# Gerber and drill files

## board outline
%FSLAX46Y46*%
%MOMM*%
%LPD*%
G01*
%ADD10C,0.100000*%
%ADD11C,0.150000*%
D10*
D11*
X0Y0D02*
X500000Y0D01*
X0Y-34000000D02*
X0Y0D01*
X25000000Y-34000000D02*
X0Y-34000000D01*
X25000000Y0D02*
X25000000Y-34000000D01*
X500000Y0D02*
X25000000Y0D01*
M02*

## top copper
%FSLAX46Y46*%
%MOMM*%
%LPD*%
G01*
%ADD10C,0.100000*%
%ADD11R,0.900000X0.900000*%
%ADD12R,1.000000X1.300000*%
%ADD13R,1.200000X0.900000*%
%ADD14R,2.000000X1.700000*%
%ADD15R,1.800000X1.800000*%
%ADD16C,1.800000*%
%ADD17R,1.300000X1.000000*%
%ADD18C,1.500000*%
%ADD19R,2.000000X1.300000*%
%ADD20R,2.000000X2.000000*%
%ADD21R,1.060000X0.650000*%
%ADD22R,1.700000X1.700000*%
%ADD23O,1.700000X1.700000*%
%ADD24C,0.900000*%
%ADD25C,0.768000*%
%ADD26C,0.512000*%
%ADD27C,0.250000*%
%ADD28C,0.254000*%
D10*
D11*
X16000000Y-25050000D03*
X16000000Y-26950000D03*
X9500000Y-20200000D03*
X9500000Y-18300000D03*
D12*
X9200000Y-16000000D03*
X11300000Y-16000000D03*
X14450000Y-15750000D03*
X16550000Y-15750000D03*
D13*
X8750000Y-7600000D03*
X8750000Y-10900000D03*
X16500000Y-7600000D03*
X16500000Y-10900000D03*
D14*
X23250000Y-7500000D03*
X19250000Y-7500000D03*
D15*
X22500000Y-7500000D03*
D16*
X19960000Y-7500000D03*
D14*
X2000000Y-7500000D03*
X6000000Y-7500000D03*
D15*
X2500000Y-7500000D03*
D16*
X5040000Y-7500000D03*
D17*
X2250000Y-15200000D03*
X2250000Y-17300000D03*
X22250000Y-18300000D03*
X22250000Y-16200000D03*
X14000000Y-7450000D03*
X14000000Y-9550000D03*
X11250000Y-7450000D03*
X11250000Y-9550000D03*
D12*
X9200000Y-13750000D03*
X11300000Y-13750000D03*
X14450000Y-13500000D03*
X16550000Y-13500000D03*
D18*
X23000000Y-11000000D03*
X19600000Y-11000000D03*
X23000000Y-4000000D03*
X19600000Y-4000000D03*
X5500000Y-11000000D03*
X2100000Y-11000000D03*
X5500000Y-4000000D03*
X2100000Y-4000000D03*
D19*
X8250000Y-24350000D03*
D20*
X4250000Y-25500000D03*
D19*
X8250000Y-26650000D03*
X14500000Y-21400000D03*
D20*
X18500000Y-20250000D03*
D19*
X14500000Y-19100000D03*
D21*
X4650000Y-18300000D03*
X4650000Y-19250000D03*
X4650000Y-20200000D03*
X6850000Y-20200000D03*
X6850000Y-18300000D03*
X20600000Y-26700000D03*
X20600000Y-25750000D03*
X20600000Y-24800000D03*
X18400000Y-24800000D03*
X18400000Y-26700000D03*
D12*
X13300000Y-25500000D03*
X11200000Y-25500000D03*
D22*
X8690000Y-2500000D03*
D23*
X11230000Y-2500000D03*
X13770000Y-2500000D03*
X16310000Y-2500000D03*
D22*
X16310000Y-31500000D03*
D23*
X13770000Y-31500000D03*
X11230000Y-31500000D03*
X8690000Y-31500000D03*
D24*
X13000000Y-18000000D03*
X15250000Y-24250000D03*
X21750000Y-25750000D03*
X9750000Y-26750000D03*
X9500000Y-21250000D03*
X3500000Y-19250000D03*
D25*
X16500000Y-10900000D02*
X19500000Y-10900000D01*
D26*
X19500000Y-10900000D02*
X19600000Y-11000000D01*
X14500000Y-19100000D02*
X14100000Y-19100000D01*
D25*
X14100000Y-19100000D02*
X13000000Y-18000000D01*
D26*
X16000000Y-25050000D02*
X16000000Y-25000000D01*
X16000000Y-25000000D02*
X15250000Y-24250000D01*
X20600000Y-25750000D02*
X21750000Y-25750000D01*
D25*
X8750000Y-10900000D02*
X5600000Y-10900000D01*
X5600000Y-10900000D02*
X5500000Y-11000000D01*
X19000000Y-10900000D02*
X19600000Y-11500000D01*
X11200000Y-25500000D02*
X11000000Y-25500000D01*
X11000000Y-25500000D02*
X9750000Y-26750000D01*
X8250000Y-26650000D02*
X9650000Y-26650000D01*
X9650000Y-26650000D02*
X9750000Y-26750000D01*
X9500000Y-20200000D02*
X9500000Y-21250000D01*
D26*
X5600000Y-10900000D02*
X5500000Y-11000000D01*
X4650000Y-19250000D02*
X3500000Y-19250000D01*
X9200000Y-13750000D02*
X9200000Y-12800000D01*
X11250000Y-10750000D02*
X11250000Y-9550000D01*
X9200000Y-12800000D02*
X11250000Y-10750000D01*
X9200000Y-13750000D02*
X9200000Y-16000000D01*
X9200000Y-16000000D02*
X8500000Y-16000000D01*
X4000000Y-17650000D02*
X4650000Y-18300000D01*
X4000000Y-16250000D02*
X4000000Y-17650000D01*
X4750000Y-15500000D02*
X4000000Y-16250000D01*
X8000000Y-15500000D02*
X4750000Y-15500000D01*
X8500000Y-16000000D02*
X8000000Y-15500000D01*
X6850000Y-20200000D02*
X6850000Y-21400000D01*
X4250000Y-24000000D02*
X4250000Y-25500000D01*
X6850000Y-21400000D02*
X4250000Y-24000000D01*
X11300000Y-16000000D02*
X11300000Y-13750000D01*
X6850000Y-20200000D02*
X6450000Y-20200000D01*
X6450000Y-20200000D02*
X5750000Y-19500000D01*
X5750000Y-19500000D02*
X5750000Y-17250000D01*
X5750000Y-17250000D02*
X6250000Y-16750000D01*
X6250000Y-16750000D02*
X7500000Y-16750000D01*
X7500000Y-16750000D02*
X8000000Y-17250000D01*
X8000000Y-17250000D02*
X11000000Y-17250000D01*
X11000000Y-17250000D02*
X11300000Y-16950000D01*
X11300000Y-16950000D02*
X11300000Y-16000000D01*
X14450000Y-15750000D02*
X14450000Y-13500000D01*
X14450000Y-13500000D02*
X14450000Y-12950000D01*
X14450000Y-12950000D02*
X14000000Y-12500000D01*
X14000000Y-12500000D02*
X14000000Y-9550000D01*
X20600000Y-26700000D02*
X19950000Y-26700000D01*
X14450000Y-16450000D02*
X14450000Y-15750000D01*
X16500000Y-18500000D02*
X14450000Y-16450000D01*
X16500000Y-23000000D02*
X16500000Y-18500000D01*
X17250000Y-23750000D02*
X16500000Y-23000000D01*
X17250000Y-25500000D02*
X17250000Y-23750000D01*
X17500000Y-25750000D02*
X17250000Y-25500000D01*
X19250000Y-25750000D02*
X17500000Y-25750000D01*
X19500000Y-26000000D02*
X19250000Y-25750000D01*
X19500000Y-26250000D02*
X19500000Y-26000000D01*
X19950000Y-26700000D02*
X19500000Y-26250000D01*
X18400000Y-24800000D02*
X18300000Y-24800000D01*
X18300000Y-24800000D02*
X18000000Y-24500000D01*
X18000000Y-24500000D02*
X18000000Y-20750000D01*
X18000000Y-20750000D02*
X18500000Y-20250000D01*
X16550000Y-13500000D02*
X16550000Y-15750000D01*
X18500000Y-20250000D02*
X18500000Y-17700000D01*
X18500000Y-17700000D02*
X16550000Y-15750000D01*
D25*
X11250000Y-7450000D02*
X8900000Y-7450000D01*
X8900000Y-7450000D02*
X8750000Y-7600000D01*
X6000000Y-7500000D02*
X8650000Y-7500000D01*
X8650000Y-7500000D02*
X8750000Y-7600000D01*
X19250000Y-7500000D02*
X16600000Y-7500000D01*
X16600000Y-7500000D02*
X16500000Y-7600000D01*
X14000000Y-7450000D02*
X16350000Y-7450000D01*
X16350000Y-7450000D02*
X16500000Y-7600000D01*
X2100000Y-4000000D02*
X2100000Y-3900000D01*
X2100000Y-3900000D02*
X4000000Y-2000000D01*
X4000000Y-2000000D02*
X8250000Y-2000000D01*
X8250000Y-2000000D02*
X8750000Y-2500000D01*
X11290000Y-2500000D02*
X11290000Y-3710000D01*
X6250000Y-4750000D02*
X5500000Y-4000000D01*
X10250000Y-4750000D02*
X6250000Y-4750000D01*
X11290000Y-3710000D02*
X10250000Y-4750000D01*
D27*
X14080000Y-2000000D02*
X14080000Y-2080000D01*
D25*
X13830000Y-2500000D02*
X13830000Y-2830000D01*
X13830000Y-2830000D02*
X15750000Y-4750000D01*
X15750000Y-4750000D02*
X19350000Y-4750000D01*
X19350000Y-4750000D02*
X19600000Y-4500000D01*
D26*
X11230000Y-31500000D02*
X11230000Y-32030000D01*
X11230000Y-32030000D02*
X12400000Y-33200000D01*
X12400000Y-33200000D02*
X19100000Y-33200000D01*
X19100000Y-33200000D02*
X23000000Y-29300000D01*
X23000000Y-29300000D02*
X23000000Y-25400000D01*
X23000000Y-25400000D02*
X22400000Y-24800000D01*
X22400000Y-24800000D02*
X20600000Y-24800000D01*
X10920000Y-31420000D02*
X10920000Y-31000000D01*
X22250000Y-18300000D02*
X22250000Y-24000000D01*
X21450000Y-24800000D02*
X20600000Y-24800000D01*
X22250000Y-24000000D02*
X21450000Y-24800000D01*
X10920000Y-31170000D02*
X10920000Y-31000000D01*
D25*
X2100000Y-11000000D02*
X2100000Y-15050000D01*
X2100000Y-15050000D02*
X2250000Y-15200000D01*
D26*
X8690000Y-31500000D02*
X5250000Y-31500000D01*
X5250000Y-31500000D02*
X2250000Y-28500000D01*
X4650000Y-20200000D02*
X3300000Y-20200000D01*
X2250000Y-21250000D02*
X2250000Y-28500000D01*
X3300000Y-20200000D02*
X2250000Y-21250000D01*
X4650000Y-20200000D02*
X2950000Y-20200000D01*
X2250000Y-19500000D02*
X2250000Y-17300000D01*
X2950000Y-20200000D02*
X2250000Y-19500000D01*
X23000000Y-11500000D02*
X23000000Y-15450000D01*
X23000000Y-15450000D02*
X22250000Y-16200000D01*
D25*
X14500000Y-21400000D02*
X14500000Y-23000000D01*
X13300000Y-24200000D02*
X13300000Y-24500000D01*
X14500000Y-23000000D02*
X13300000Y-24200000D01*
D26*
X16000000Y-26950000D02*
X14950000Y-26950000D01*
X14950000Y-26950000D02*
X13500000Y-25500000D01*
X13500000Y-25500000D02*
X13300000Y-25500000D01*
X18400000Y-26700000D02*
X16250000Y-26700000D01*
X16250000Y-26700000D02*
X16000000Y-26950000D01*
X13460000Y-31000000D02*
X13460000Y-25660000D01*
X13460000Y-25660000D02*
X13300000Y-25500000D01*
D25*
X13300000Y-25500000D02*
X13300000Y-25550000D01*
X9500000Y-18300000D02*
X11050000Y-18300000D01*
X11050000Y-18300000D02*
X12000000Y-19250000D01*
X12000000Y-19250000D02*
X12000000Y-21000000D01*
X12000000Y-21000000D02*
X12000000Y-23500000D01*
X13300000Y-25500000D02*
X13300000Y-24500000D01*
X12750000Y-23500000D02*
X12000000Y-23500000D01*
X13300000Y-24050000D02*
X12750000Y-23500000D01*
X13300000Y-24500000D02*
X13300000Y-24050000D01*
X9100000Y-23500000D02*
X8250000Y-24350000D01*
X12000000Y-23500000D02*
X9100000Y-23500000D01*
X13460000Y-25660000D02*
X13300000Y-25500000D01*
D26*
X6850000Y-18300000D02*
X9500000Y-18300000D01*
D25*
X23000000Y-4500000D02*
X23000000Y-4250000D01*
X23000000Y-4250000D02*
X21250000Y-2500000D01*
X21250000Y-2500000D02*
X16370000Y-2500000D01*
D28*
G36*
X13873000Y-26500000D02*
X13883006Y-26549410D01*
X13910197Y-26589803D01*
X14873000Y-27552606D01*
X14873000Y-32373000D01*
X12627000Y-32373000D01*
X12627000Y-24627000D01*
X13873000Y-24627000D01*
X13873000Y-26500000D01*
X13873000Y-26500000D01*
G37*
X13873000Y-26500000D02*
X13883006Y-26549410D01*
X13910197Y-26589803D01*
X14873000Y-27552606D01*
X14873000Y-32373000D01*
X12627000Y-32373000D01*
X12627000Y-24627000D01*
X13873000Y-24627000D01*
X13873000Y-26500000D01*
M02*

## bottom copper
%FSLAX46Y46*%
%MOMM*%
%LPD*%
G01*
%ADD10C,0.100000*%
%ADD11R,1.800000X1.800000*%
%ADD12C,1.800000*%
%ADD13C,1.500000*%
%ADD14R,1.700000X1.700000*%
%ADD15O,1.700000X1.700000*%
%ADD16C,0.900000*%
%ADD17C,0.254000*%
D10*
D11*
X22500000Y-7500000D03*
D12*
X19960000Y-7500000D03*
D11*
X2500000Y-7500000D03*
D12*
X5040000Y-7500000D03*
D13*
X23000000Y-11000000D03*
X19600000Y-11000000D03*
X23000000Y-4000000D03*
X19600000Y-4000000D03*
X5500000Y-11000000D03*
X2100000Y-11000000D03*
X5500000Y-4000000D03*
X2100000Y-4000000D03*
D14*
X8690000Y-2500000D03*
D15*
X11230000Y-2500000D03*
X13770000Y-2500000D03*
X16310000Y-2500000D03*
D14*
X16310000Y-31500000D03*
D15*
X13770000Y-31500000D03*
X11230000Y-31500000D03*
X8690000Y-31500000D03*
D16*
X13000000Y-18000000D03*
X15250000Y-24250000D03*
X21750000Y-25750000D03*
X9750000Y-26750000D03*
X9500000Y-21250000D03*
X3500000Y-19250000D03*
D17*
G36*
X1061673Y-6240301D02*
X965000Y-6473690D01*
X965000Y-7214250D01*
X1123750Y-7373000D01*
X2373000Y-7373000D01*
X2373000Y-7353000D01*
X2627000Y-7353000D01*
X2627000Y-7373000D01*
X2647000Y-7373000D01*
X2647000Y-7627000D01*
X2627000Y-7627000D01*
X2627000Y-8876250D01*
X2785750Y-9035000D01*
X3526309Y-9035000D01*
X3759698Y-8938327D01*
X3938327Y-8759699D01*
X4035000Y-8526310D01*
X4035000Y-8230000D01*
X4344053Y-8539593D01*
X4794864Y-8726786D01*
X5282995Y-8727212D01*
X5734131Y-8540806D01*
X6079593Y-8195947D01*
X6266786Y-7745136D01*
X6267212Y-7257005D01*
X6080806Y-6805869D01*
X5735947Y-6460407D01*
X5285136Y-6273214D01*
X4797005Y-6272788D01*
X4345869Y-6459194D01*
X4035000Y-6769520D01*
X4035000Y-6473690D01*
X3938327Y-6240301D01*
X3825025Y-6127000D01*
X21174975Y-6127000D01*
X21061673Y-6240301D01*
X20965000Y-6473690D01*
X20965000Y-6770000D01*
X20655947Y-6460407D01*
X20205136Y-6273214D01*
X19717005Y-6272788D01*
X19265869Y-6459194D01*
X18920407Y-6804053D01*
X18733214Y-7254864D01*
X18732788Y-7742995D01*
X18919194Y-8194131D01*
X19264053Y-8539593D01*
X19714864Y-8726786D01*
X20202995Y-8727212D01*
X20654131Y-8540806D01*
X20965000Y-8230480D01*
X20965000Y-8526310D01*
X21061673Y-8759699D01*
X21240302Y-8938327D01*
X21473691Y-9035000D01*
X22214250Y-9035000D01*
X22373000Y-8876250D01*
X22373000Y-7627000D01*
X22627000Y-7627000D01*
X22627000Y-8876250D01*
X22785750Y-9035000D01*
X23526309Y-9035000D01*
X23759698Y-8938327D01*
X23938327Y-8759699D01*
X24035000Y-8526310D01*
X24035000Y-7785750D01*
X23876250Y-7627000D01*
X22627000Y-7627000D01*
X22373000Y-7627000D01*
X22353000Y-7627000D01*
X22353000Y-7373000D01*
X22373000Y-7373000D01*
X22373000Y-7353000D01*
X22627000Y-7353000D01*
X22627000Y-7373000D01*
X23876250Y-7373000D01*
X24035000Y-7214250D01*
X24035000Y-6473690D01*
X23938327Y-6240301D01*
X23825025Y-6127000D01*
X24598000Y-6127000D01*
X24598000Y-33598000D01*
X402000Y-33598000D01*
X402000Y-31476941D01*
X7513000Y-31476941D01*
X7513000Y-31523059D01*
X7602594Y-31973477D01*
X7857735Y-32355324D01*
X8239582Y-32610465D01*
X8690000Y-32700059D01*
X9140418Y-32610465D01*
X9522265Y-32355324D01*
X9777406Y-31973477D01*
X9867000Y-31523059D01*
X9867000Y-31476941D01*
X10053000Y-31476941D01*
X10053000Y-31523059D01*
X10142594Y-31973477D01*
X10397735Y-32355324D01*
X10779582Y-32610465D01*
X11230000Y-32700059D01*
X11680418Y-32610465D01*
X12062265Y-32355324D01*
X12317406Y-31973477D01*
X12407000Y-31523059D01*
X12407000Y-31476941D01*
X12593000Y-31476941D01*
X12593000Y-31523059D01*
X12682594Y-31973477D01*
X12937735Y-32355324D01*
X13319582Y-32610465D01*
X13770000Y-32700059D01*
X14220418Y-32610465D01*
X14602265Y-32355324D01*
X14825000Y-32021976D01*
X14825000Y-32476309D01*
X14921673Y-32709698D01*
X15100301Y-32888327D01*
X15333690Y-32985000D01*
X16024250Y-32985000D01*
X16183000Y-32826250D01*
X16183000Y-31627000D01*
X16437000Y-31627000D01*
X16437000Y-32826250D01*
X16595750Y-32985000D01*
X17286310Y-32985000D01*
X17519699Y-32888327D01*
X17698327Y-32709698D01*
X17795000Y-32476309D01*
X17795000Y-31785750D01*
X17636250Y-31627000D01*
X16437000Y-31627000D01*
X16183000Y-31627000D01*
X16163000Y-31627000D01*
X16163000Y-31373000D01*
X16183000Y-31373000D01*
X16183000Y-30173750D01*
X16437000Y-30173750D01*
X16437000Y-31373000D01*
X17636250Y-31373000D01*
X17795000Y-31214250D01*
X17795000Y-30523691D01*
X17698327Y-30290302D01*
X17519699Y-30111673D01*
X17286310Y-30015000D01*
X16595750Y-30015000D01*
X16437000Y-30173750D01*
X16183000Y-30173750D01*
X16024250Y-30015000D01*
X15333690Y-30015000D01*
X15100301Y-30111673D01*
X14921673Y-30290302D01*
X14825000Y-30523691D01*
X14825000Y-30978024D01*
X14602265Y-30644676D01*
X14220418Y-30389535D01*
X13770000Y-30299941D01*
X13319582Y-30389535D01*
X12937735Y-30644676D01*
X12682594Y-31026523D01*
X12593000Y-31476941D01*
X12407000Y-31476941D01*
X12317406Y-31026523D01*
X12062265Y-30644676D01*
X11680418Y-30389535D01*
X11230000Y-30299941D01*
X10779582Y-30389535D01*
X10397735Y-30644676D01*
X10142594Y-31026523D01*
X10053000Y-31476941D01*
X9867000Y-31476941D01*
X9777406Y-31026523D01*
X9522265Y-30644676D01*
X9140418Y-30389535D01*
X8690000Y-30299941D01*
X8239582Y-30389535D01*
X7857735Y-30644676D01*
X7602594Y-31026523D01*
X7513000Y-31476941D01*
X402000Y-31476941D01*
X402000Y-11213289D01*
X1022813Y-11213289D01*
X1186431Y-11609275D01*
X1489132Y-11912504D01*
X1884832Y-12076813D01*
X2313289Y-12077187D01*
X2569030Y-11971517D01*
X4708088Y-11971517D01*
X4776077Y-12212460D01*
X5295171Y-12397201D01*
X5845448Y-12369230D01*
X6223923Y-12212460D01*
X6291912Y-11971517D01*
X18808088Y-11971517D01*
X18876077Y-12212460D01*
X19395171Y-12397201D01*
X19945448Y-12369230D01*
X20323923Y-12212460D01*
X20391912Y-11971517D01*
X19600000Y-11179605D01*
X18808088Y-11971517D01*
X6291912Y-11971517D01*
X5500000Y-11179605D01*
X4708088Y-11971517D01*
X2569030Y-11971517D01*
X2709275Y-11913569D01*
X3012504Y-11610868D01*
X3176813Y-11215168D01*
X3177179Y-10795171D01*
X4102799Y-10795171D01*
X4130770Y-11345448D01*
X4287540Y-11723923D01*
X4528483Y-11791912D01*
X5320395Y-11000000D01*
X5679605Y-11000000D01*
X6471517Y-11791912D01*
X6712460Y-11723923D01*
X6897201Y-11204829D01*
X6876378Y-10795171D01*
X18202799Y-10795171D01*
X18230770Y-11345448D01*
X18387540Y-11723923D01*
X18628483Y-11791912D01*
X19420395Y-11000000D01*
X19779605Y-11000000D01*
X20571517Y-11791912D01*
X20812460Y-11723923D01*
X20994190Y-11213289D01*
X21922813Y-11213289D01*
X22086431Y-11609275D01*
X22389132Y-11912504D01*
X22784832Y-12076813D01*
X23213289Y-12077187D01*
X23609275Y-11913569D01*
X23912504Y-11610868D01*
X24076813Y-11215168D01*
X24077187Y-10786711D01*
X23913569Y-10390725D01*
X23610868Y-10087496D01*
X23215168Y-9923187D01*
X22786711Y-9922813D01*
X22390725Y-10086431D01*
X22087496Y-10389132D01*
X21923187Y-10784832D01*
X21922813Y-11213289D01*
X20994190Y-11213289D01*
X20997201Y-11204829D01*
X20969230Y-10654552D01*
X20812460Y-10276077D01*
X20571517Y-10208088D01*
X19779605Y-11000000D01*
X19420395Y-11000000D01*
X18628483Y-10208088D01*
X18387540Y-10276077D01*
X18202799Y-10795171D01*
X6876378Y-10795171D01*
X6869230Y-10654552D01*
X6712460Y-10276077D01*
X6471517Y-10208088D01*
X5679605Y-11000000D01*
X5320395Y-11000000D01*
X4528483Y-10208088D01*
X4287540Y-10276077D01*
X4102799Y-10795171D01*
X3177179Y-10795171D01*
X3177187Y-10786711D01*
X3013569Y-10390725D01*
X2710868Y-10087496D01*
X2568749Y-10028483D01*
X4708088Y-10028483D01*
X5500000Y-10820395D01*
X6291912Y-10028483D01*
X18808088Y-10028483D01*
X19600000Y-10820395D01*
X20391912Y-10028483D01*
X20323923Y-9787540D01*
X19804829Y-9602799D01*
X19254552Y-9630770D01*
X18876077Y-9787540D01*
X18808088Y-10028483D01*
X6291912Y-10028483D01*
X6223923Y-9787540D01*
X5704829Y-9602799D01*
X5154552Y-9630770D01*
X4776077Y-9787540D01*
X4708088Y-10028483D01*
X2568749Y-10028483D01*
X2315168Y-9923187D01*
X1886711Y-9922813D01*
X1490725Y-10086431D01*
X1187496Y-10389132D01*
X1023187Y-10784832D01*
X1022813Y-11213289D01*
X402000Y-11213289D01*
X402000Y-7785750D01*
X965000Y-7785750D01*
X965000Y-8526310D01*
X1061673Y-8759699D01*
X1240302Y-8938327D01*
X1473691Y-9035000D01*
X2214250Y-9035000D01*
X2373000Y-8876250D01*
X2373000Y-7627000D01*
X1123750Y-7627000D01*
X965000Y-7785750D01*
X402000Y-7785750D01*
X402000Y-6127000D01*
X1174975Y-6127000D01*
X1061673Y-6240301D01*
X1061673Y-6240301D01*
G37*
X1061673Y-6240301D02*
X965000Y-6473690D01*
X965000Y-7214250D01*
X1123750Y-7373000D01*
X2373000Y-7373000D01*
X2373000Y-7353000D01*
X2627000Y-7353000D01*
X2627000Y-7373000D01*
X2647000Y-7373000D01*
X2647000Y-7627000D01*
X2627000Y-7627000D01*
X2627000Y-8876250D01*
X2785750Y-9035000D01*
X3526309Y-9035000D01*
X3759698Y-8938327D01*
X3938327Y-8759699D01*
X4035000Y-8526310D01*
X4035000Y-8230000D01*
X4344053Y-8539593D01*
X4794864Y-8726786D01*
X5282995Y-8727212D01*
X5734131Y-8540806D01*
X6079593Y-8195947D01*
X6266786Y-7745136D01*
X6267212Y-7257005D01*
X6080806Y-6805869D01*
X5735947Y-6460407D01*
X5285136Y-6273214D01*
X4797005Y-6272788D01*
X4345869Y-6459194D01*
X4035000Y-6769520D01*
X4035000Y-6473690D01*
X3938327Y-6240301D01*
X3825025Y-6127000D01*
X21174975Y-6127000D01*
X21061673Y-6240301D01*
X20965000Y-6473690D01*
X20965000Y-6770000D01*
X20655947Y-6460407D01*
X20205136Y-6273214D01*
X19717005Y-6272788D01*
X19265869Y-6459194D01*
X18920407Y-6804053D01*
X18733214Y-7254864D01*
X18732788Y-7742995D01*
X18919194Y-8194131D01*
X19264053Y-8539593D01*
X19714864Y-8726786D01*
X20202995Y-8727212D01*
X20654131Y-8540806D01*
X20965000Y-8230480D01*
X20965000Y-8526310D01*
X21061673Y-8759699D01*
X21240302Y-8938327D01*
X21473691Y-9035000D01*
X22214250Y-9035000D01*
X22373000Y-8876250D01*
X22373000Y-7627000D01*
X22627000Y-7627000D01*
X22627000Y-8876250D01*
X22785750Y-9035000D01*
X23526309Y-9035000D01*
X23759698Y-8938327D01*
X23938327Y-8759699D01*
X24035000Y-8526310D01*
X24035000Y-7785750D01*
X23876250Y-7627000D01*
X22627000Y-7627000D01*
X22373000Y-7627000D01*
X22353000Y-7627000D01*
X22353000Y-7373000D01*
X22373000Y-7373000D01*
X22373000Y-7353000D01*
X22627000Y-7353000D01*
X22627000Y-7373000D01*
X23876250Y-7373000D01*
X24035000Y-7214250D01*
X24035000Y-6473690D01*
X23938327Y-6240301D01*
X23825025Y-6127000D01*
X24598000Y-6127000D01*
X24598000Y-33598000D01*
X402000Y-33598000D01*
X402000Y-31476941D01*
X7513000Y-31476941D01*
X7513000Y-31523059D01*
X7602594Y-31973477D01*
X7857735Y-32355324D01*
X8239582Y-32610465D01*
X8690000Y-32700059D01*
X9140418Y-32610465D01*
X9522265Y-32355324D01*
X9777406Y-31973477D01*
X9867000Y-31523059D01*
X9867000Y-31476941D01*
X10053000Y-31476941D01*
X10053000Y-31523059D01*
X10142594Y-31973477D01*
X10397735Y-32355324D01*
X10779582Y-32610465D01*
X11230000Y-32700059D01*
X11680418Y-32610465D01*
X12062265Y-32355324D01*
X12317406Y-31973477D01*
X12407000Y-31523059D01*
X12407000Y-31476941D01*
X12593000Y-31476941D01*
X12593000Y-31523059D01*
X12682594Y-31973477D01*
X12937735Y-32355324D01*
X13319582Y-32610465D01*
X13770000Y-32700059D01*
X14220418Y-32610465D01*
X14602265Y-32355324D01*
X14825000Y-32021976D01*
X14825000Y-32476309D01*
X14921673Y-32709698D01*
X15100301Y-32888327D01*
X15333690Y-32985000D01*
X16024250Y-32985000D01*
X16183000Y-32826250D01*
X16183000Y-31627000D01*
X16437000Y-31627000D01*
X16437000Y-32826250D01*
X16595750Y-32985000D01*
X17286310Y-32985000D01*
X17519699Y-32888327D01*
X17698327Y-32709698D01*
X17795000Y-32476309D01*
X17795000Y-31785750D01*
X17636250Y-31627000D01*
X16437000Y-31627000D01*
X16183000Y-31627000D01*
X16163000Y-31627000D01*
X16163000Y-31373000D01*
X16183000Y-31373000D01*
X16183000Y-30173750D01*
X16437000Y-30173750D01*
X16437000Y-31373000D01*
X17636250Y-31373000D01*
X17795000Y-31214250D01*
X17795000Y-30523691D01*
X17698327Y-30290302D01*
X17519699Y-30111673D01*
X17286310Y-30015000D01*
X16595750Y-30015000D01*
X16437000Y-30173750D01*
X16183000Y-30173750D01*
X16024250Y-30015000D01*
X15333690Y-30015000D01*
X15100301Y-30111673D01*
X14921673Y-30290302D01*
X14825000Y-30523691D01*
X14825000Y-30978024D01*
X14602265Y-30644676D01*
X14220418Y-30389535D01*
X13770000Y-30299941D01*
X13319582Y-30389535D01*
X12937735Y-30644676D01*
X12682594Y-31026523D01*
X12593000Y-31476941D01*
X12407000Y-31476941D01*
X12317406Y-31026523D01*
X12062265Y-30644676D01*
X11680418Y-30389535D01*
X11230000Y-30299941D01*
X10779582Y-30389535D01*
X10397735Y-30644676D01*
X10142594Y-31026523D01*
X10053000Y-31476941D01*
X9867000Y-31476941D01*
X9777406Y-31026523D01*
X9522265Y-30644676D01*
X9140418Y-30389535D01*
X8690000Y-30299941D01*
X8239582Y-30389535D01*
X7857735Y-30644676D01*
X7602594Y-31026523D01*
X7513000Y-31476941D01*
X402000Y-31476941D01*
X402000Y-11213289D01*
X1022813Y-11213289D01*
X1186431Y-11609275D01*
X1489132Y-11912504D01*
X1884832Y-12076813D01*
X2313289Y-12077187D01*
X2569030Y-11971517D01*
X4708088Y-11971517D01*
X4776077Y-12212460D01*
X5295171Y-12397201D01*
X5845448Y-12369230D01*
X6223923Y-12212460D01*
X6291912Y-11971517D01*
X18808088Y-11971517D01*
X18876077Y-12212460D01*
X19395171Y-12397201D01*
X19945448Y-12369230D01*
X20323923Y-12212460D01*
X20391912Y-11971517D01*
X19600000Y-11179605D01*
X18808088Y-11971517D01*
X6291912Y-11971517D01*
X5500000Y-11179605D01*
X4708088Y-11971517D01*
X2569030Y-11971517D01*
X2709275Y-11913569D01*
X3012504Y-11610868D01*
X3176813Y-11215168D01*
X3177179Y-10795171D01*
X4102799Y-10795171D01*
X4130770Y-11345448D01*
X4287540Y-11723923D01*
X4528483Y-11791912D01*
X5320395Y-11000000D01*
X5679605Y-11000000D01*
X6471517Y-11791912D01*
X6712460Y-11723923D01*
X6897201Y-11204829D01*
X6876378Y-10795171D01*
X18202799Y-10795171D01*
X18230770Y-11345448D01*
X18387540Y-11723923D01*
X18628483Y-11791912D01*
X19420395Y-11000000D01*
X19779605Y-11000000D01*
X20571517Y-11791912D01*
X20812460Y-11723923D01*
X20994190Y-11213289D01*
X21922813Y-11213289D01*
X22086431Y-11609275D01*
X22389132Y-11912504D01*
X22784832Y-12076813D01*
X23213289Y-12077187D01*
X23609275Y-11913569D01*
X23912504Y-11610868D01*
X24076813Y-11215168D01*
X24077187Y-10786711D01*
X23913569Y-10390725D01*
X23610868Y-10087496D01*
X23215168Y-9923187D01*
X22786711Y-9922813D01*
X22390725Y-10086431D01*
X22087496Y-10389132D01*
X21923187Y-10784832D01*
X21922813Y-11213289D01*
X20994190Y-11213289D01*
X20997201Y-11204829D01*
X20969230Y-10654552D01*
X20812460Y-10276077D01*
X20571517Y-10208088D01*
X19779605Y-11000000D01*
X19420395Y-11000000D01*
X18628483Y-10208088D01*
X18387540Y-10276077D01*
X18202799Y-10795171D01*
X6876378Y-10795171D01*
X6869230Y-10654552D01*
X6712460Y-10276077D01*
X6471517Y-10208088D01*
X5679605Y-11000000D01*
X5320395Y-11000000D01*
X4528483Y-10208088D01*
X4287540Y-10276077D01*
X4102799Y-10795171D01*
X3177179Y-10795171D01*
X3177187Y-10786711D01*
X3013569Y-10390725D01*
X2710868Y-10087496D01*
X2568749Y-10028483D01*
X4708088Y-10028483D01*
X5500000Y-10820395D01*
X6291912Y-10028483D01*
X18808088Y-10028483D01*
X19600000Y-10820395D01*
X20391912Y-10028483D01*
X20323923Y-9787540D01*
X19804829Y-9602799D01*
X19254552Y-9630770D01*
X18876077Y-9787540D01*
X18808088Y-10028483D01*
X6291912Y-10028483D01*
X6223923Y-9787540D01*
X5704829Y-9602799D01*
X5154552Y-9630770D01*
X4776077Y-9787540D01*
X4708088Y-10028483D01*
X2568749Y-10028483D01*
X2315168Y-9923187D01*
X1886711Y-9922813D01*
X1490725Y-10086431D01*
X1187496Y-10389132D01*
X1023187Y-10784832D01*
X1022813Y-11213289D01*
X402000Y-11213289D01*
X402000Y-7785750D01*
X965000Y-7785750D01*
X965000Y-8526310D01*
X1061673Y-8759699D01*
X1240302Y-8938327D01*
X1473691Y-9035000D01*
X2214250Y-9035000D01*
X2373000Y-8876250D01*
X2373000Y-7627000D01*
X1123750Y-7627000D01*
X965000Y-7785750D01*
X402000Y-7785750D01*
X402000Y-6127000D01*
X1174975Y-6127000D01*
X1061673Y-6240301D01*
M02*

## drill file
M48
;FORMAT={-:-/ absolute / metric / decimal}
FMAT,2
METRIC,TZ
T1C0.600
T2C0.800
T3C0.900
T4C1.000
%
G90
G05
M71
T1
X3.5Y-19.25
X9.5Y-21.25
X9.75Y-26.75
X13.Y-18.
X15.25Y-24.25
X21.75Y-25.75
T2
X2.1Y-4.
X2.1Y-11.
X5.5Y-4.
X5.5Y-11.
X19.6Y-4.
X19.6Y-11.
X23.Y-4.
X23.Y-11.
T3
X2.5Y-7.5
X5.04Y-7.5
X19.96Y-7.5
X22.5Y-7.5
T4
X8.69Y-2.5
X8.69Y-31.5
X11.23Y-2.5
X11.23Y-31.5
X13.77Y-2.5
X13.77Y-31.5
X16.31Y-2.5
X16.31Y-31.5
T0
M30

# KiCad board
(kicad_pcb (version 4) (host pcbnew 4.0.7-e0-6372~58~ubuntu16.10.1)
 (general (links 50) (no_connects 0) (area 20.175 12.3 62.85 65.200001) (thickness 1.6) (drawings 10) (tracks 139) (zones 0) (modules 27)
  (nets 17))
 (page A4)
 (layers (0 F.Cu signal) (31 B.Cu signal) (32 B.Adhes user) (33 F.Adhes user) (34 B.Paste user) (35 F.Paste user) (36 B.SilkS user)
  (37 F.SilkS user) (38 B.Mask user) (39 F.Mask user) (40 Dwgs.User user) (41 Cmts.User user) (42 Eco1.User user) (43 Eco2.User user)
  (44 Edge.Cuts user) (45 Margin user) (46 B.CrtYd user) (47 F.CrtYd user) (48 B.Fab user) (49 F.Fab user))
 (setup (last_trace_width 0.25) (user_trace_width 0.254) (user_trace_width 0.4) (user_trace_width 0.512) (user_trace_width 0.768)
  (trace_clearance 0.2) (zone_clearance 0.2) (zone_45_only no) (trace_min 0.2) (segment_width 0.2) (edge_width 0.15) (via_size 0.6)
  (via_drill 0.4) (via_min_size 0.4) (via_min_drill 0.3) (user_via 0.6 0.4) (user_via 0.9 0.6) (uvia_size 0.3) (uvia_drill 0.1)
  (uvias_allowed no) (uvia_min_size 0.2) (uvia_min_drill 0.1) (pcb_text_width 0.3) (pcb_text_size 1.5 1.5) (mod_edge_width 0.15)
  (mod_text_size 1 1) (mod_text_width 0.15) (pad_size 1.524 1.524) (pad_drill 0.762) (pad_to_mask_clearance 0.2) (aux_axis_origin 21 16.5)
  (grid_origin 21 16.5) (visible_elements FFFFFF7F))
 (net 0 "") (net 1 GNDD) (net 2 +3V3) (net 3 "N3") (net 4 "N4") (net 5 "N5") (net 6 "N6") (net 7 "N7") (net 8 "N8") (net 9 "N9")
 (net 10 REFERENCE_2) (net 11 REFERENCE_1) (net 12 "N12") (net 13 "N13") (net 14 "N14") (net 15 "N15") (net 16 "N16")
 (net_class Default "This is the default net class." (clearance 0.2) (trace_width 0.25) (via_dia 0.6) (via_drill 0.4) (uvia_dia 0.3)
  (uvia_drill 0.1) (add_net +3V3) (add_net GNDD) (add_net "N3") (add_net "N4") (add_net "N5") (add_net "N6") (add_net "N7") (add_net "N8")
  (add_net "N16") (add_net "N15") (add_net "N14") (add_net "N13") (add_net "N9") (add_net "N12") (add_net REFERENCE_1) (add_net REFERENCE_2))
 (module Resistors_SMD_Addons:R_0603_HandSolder (layer F.Cu) (at 37 42.5 270)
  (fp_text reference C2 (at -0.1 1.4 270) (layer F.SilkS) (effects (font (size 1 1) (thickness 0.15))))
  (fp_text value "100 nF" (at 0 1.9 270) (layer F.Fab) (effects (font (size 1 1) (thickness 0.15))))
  (pad 1 smd rect (at -0.95 0 270) (size 0.9 0.9) (layers F.Cu F.Paste F.Mask) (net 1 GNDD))
  (pad 2 smd rect (at 0.95 0 270) (size 0.9 0.9) (layers F.Cu F.Paste F.Mask) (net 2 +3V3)))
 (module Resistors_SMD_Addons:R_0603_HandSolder (layer F.Cu) (at 30.5 35.75 90)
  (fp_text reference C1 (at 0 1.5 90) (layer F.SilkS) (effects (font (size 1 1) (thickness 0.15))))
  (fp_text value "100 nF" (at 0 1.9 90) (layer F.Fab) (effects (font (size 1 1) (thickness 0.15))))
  (pad 1 smd rect (at -0.95 0 90) (size 0.9 0.9) (layers F.Cu F.Paste F.Mask) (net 1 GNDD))
  (pad 2 smd rect (at 0.95 0 90) (size 0.9 0.9) (layers F.Cu F.Paste F.Mask) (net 2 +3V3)))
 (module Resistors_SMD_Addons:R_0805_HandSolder (layer F.Cu) (at 31.25 32.5)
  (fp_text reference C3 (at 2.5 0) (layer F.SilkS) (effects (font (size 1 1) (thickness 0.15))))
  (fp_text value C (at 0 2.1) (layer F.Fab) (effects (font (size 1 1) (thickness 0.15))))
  (pad 1 smd rect (at -1.05 0) (size 1 1.3) (layers F.Cu F.Paste F.Mask) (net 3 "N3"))
  (pad 2 smd rect (at 1.05 0) (size 1 1.3) (layers F.Cu F.Paste F.Mask) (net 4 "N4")))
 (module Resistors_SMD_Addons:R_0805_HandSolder (layer F.Cu) (at 36.5 32.25)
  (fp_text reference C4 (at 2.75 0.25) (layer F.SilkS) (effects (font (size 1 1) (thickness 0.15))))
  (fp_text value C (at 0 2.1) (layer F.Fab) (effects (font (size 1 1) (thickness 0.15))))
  (pad 1 smd rect (at -1.05 0) (size 1 1.3) (layers F.Cu F.Paste F.Mask) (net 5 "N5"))
  (pad 2 smd rect (at 1.05 0) (size 1 1.3) (layers F.Cu F.Paste F.Mask) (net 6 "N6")))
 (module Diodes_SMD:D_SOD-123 (layer F.Cu) (at 29.75 25.75 270)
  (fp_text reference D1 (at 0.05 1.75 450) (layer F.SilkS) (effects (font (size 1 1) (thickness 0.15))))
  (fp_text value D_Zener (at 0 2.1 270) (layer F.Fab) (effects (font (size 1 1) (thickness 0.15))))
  (pad 1 smd rect (at -1.65 0 270) (size 0.9 1.2) (layers F.Cu F.Paste F.Mask) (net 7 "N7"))
  (pad 2 smd rect (at 1.65 0 270) (size 0.9 1.2) (layers F.Cu F.Paste F.Mask) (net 1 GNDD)))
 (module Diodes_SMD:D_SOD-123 (layer F.Cu) (at 37.5 25.75 270)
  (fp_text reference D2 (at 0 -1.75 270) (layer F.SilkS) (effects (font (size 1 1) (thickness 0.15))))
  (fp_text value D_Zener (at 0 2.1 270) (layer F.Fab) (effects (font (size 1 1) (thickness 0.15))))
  (pad 1 smd rect (at -1.65 0 270) (size 0.9 1.2) (layers F.Cu F.Paste F.Mask) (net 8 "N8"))
  (pad 2 smd rect (at 1.65 0 270) (size 0.9 1.2) (layers F.Cu F.Paste F.Mask) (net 1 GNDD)))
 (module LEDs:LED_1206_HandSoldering (layer F.Cu) (at 42.25 24 180)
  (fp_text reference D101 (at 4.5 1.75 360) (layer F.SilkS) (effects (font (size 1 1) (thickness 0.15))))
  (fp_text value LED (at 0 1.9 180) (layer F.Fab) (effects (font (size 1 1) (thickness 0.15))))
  (pad 1 smd rect (at -2 0 180) (size 2 1.7) (layers F.Cu F.Paste F.Mask) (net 1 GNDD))
  (pad 2 smd rect (at 2 0 180) (size 2 1.7) (layers F.Cu F.Paste F.Mask) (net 8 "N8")))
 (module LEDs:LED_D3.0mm (layer F.Cu) (at 43.5 24 180)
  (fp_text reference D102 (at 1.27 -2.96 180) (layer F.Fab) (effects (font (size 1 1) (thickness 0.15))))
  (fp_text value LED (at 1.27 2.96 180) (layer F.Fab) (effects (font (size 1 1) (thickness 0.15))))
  (pad 1 thru_hole rect (at 0 0 180) (size 1.8 1.8) (drill 0.9) (layers *.Cu *.Mask) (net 1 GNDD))
  (pad 2 thru_hole circle (at 2.54 0 180) (size 1.8 1.8) (drill 0.9) (layers *.Cu *.Mask) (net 8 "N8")))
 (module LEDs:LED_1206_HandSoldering (layer F.Cu) (at 25 24)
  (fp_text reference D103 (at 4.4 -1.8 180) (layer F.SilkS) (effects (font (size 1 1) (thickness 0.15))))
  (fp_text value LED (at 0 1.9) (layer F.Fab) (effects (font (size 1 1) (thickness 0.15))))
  (pad 1 smd rect (at -2 0) (size 2 1.7) (layers F.Cu F.Paste F.Mask) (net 1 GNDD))
  (pad 2 smd rect (at 2 0) (size 2 1.7) (layers F.Cu F.Paste F.Mask) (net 7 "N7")))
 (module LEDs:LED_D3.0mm (layer F.Cu) (at 23.5 24)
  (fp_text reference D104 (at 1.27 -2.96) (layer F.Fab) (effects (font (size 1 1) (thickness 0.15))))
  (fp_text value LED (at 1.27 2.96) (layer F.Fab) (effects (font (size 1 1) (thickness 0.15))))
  (pad 1 thru_hole rect (at 0 0) (size 1.8 1.8) (drill 0.9) (layers *.Cu *.Mask) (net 1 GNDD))
  (pad 2 thru_hole circle (at 2.54 0) (size 1.8 1.8) (drill 0.9) (layers *.Cu *.Mask) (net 7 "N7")))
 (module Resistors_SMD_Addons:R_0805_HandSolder (layer F.Cu) (at 23.25 32.75 270)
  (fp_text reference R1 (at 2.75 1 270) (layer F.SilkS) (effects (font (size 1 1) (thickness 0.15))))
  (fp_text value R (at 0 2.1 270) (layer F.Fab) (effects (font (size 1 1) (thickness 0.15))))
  (pad 1 smd rect (at -1.05 0 270) (size 1 1.3) (layers F.Cu F.Paste F.Mask) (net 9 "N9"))
  (pad 2 smd rect (at 1.05 0 270) (size 1 1.3) (layers F.Cu F.Paste F.Mask) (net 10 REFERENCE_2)))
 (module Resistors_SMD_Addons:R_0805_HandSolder (layer F.Cu) (at 43.25 33.75 90)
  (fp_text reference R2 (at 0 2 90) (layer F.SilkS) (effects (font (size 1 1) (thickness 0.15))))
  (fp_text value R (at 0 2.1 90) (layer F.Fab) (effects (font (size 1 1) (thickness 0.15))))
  (pad 1 smd rect (at -1.05 0 90) (size 1 1.3) (layers F.Cu F.Paste F.Mask) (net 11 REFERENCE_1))
  (pad 2 smd rect (at 1.05 0 90) (size 1 1.3) (layers F.Cu F.Paste F.Mask) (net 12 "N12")))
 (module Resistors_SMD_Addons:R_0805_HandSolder (layer F.Cu) (at 35 25 270)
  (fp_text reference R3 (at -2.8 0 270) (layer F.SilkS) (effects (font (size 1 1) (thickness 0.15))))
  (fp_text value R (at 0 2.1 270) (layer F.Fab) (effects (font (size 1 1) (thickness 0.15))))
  (pad 1 smd rect (at -1.05 0 270) (size 1 1.3) (layers F.Cu F.Paste F.Mask) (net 8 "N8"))
  (pad 2 smd rect (at 1.05 0 270) (size 1 1.3) (layers F.Cu F.Paste F.Mask) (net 5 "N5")))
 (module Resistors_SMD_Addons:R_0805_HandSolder (layer F.Cu) (at 32.25 25 270)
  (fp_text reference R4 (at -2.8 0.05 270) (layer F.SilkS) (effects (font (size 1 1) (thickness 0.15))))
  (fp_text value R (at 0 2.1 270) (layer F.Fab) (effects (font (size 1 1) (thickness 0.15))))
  (pad 1 smd rect (at -1.05 0 270) (size 1 1.3) (layers F.Cu F.Paste F.Mask) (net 7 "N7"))
  (pad 2 smd rect (at 1.05 0 270) (size 1 1.3) (layers F.Cu F.Paste F.Mask) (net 3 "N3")))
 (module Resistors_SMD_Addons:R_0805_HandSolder (layer F.Cu) (at 31.25 30.25)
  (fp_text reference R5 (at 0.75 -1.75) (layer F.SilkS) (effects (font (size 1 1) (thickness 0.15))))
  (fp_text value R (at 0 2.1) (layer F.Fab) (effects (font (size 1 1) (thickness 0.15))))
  (pad 1 smd rect (at -1.05 0) (size 1 1.3) (layers F.Cu F.Paste F.Mask) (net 3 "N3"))
  (pad 2 smd rect (at 1.05 0) (size 1 1.3) (layers F.Cu F.Paste F.Mask) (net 4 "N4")))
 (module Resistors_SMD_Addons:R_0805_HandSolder (layer F.Cu) (at 36.5 30)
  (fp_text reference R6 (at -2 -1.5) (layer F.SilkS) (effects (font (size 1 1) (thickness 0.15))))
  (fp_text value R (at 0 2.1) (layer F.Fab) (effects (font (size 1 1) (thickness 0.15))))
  (pad 1 smd rect (at -1.05 0) (size 1 1.3) (layers F.Cu F.Paste F.Mask) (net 5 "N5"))
  (pad 2 smd rect (at 1.05 0) (size 1 1.3) (layers F.Cu F.Paste F.Mask) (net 6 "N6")))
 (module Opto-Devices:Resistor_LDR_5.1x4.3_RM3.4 (layer F.Cu) (at 44 27.5 180)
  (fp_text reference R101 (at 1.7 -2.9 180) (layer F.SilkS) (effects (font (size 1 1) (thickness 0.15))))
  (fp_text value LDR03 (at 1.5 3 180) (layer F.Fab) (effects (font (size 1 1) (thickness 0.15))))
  (pad 1 thru_hole circle (at 0 0 180) (size 1.5 1.5) (drill 0.8) (layers *.Cu *.Mask) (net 12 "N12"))
  (pad 2 thru_hole circle (at 3.4 0 180) (size 1.5 1.5) (drill 0.8) (layers *.Cu *.Mask) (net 1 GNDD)))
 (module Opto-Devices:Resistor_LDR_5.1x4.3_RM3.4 (layer F.Cu) (at 44 20.5 180)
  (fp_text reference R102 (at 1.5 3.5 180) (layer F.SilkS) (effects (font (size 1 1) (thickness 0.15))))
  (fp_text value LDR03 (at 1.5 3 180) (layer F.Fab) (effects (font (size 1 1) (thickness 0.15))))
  (pad 1 thru_hole circle (at 0 0 180) (size 1.5 1.5) (drill 0.8) (layers *.Cu *.Mask) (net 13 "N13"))
  (pad 2 thru_hole circle (at 3.4 0 180) (size 1.5 1.5) (drill 0.8) (layers *.Cu *.Mask) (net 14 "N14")))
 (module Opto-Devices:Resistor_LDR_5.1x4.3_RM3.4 (layer F.Cu) (at 26.5 27.5 180)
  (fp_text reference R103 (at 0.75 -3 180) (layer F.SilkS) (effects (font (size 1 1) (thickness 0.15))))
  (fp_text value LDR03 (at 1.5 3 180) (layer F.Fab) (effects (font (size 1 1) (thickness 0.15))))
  (pad 1 thru_hole circle (at 0 0 180) (size 1.5 1.5) (drill 0.8) (layers *.Cu *.Mask) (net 1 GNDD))
  (pad 2 thru_hole circle (at 3.4 0 180) (size 1.5 1.5) (drill 0.8) (layers *.Cu *.Mask) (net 9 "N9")))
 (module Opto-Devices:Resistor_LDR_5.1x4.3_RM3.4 (layer F.Cu) (at 26.5 20.5 180)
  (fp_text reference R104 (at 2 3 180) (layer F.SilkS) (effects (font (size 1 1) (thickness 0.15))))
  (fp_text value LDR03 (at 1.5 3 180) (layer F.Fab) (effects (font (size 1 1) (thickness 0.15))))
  (pad 1 thru_hole circle (at 0 0 180) (size 1.5 1.5) (drill 0.8) (layers *.Cu *.Mask) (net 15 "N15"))
  (pad 2 thru_hole circle (at 3.4 0 180) (size 1.5 1.5) (drill 0.8) (layers *.Cu *.Mask) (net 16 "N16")))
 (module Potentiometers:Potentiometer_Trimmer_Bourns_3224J (layer F.Cu) (at 27.25 42)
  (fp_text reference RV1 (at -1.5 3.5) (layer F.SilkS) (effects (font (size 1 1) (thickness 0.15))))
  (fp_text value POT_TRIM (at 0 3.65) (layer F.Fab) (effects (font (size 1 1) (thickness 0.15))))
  (pad 1 smd rect (at 2 -1.15) (size 2 1.3) (layers F.Cu F.Mask) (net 2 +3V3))
  (pad 2 smd rect (at -2 0) (size 2 2) (layers F.Cu F.Mask) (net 4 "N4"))
  (pad 3 smd rect (at 2 1.15) (size 2 1.3) (layers F.Cu F.Mask) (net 1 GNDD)))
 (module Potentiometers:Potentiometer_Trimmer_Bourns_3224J (layer F.Cu) (at 37.5 36.75 180)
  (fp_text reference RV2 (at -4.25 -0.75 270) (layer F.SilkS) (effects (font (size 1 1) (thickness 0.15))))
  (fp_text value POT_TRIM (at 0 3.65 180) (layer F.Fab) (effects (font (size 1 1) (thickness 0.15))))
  (pad 1 smd rect (at 2 -1.15 180) (size 2 1.3) (layers F.Cu F.Mask) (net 2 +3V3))
  (pad 2 smd rect (at -2 0 180) (size 2 2) (layers F.Cu F.Mask) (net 6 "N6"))
  (pad 3 smd rect (at 2 1.15 180) (size 2 1.3) (layers F.Cu F.Mask) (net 1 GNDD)))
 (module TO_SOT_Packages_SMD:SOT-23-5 (layer F.Cu) (at 26.75 35.75)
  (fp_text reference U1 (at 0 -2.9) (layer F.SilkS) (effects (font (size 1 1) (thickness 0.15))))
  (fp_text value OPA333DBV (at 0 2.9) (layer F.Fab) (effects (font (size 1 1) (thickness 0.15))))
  (pad 1 smd rect (at -1.1 -0.95) (size 1.06 0.65) (layers F.Cu F.Paste F.Mask) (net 3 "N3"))
  (pad 2 smd rect (at -1.1 0) (size 1.06 0.65) (layers F.Cu F.Paste F.Mask) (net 1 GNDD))
  (pad 3 smd rect (at -1.1 0.95) (size 1.06 0.65) (layers F.Cu F.Paste F.Mask) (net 10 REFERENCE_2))
  (pad 4 smd rect (at 1.1 0.95) (size 1.06 0.65) (layers F.Cu F.Paste F.Mask) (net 4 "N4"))
  (pad 5 smd rect (at 1.1 -0.95) (size 1.06 0.65) (layers F.Cu F.Paste F.Mask) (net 2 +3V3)))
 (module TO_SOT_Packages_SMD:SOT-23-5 (layer F.Cu) (at 40.5 42.25 180)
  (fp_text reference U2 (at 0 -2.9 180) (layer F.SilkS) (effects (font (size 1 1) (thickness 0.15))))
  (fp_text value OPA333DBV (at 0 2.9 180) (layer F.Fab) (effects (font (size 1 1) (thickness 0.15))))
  (pad 1 smd rect (at -1.1 -0.95 180) (size 1.06 0.65) (layers F.Cu F.Paste F.Mask) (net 5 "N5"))
  (pad 2 smd rect (at -1.1 0 180) (size 1.06 0.65) (layers F.Cu F.Paste F.Mask) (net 1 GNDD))
  (pad 3 smd rect (at -1.1 0.95 180) (size 1.06 0.65) (layers F.Cu F.Paste F.Mask) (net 11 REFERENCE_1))
  (pad 4 smd rect (at 1.1 0.95 180) (size 1.06 0.65) (layers F.Cu F.Paste F.Mask) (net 6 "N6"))
  (pad 5 smd rect (at 1.1 -0.95 180) (size 1.06 0.65) (layers F.Cu F.Paste F.Mask) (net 2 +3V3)))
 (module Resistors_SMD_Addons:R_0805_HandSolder (layer F.Cu) (at 33.25 42 180)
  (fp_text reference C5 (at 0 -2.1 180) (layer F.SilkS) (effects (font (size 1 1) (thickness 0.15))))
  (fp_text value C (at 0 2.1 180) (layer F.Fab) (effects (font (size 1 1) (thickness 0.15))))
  (pad 1 smd rect (at -1.05 0 180) (size 1 1.3) (layers F.Cu F.Paste F.Mask) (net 2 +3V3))
  (pad 2 smd rect (at 1.05 0 180) (size 1 1.3) (layers F.Cu F.Paste F.Mask) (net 1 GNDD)))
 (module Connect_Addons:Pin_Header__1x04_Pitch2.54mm (layer B.Cu) (at 33.5 19)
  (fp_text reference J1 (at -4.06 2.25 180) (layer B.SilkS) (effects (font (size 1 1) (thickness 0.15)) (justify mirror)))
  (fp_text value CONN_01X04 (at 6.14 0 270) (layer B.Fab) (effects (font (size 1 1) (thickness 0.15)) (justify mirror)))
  (pad 1 thru_hole rect (at -3.81 0 270) (size 1.7 1.7) (drill 1) (layers *.Cu *.Mask) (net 16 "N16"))
  (pad 2 thru_hole oval (at -1.27 0 270) (size 1.7 1.7) (drill 1) (layers *.Cu *.Mask) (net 15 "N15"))
  (pad 3 thru_hole oval (at 1.27 0 270) (size 1.7 1.7) (drill 1) (layers *.Cu *.Mask) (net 14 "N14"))
  (pad 4 thru_hole oval (at 3.81 0 270) (size 1.7 1.7) (drill 1) (layers *.Cu *.Mask) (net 13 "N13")))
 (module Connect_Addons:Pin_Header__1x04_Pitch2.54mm (layer B.Cu) (at 33.5 48 180)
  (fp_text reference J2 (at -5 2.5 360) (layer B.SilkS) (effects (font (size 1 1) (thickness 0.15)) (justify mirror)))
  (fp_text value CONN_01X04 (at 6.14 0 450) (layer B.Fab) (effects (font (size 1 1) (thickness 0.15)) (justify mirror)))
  (pad 1 thru_hole rect (at -3.81 0 90) (size 1.7 1.7) (drill 1) (layers *.Cu *.Mask) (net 1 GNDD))
  (pad 2 thru_hole oval (at -1.27 0 90) (size 1.7 1.7) (drill 1) (layers *.Cu *.Mask) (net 2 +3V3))
  (pad 3 thru_hole oval (at 1.27 0 90) (size 1.7 1.7) (drill 1) (layers *.Cu *.Mask) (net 11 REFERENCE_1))
  (pad 4 thru_hole oval (at 3.81 0 90) (size 1.7 1.7) (drill 1) (layers *.Cu *.Mask) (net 10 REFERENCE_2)))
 (gr_line (start 21 16.5) (end 21.5 16.5) (angle 90) (layer Edge.Cuts) (width 0.15))
 (gr_line (start 21 50.5) (end 21 16.5) (angle 90) (layer Edge.Cuts) (width 0.15))
 (gr_line (start 46 50.5) (end 21 50.5) (angle 90) (layer Edge.Cuts) (width 0.15))
 (gr_line (start 46 16.5) (end 46 50.5) (angle 90) (layer Edge.Cuts) (width 0.15))
 (gr_line (start 21.5 16.5) (end 46 16.5) (angle 90) (layer Edge.Cuts) (width 0.15))
 (segment (start 37.5 27.4) (end 40.5 27.4) (width 0.768) (layer F.Cu) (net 1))
 (segment (start 40.5 27.4) (end 40.6 27.5) (width 0.512) (layer F.Cu) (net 1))
 (segment (start 35.5 35.6) (end 35.1 35.6) (width 0.512) (layer F.Cu) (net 1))
 (segment (start 35.1 35.6) (end 34 34.5) (width 0.768) (layer F.Cu) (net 1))
 (via (at 34 34.5) (size 0.9) (drill 0.6) (layers F.Cu B.Cu) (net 1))
 (segment (start 37 41.55) (end 37 41.5) (width 0.512) (layer F.Cu) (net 1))
 (segment (start 37 41.5) (end 36.25 40.75) (width 0.512) (layer F.Cu) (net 1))
 (via (at 36.25 40.75) (size 0.9) (drill 0.6) (layers F.Cu B.Cu) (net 1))
 (segment (start 41.6 42.25) (end 42.75 42.25) (width 0.512) (layer F.Cu) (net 1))
 (via (at 42.75 42.25) (size 0.9) (drill 0.6) (layers F.Cu B.Cu) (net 1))
 (segment (start 29.75 27.4) (end 26.6 27.4) (width 0.768) (layer F.Cu) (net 1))
 (segment (start 26.6 27.4) (end 26.5 27.5) (width 0.768) (layer F.Cu) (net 1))
 (segment (start 40 27.4) (end 40.6 28) (width 0.768) (layer F.Cu) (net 1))
 (segment (start 32.2 42) (end 32 42) (width 0.768) (layer F.Cu) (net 1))
 (segment (start 32 42) (end 30.75 43.25) (width 0.768) (layer F.Cu) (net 1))
 (segment (start 29.25 43.15) (end 30.65 43.15) (width 0.768) (layer F.Cu) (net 1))
 (via (at 30.75 43.25) (size 0.9) (drill 0.6) (layers F.Cu B.Cu) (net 1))
 (segment (start 30.65 43.15) (end 30.75 43.25) (width 0.768) (layer F.Cu) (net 1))
 (segment (start 30.5 36.7) (end 30.5 37.75) (width 0.768) (layer F.Cu) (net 1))
 (via (at 30.5 37.75) (size 0.9) (drill 0.6) (layers F.Cu B.Cu) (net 1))
 (segment (start 26.6 27.4) (end 26.5 27.5) (width 0.512) (layer F.Cu) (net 1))
 (segment (start 25.65 35.75) (end 24.5 35.75) (width 0.512) (layer F.Cu) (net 1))
 (via (at 24.5 35.75) (size 0.9) (drill 0.6) (layers F.Cu B.Cu) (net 1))
 (segment (start 30.2 30.25) (end 30.2 29.3) (width 0.512) (layer F.Cu) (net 3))
 (segment (start 32.25 27.25) (end 32.25 26.05) (width 0.512) (layer F.Cu) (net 3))
 (segment (start 30.2 29.3) (end 32.25 27.25) (width 0.512) (layer F.Cu) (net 3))
 (segment (start 30.2 30.25) (end 30.2 32.5) (width 0.512) (layer F.Cu) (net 3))
 (segment (start 30.2 32.5) (end 29.5 32.5) (width 0.512) (layer F.Cu) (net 3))
 (segment (start 25 34.15) (end 25.65 34.8) (width 0.512) (layer F.Cu) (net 3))
 (segment (start 25 32.75) (end 25 34.15) (width 0.512) (layer F.Cu) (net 3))
 (segment (start 25.75 32) (end 25 32.75) (width 0.512) (layer F.Cu) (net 3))
 (segment (start 29 32) (end 25.75 32) (width 0.512) (layer F.Cu) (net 3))
 (segment (start 29.5 32.5) (end 29 32) (width 0.512) (layer F.Cu) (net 3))
 (segment (start 27.85 36.7) (end 27.85 37.9) (width 0.512) (layer F.Cu) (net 4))
 (segment (start 25.25 40.5) (end 25.25 42) (width 0.512) (layer F.Cu) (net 4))
 (segment (start 27.85 37.9) (end 25.25 40.5) (width 0.512) (layer F.Cu) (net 4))
 (segment (start 32.3 32.5) (end 32.3 30.25) (width 0.512) (layer F.Cu) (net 4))
 (segment (start 27.85 36.7) (end 27.45 36.7) (width 0.512) (layer F.Cu) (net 4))
 (segment (start 27.45 36.7) (end 26.75 36) (width 0.512) (layer F.Cu) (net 4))
 (segment (start 26.75 36) (end 26.75 33.75) (width 0.512) (layer F.Cu) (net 4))
 (segment (start 26.75 33.75) (end 27.25 33.25) (width 0.512) (layer F.Cu) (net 4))
 (segment (start 27.25 33.25) (end 28.5 33.25) (width 0.512) (layer F.Cu) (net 4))
 (segment (start 28.5 33.25) (end 29 33.75) (width 0.512) (layer F.Cu) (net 4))
 (segment (start 29 33.75) (end 32 33.75) (width 0.512) (layer F.Cu) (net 4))
 (segment (start 32 33.75) (end 32.3 33.45) (width 0.512) (layer F.Cu) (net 4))
 (segment (start 32.3 33.45) (end 32.3 32.5) (width 0.512) (layer F.Cu) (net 4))
 (segment (start 35.45 32.25) (end 35.45 30) (width 0.512) (layer F.Cu) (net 5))
 (segment (start 35.45 30) (end 35.45 29.45) (width 0.512) (layer F.Cu) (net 5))
 (segment (start 35.45 29.45) (end 35 29) (width 0.512) (layer F.Cu) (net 5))
 (segment (start 35 29) (end 35 26.05) (width 0.512) (layer F.Cu) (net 5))
 (segment (start 41.6 43.2) (end 40.95 43.2) (width 0.512) (layer F.Cu) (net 5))
 (segment (start 35.45 32.95) (end 35.45 32.25) (width 0.512) (layer F.Cu) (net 5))
 (segment (start 37.5 35) (end 35.45 32.95) (width 0.512) (layer F.Cu) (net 5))
 (segment (start 37.5 39.5) (end 37.5 35) (width 0.512) (layer F.Cu) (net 5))
 (segment (start 38.25 40.25) (end 37.5 39.5) (width 0.512) (layer F.Cu) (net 5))
 (segment (start 38.25 42) (end 38.25 40.25) (width 0.512) (layer F.Cu) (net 5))
 (segment (start 38.5 42.25) (end 38.25 42) (width 0.512) (layer F.Cu) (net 5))
 (segment (start 40.25 42.25) (end 38.5 42.25) (width 0.512) (layer F.Cu) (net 5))
 (segment (start 40.5 42.5) (end 40.25 42.25) (width 0.512) (layer F.Cu) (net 5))
 (segment (start 40.5 42.75) (end 40.5 42.5) (width 0.512) (layer F.Cu) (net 5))
 (segment (start 40.95 43.2) (end 40.5 42.75) (width 0.512) (layer F.Cu) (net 5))
 (segment (start 39.4 41.3) (end 39.3 41.3) (width 0.512) (layer F.Cu) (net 6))
 (segment (start 39.3 41.3) (end 39 41) (width 0.512) (layer F.Cu) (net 6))
 (segment (start 39 41) (end 39 37.25) (width 0.512) (layer F.Cu) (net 6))
 (segment (start 39 37.25) (end 39.5 36.75) (width 0.512) (layer F.Cu) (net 6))
 (segment (start 37.55 30) (end 37.55 32.25) (width 0.512) (layer F.Cu) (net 6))
 (segment (start 39.5 36.75) (end 39.5 34.2) (width 0.512) (layer F.Cu) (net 6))
 (segment (start 39.5 34.2) (end 37.55 32.25) (width 0.512) (layer F.Cu) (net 6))
 (segment (start 32.25 23.95) (end 29.9 23.95) (width 0.768) (layer F.Cu) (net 7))
 (segment (start 29.9 23.95) (end 29.75 24.1) (width 0.768) (layer F.Cu) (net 7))
 (segment (start 27 24) (end 29.65 24) (width 0.768) (layer F.Cu) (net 7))
 (segment (start 29.65 24) (end 29.75 24.1) (width 0.768) (layer F.Cu) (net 7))
 (segment (start 40.25 24) (end 37.6 24) (width 0.768) (layer F.Cu) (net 8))
 (segment (start 37.6 24) (end 37.5 24.1) (width 0.768) (layer F.Cu) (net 8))
 (segment (start 35 23.95) (end 37.35 23.95) (width 0.768) (layer F.Cu) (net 8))
 (segment (start 37.35 23.95) (end 37.5 24.1) (width 0.768) (layer F.Cu) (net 8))
 (segment (start 23.1 20.5) (end 23.1 20.4) (width 0.768) (layer F.Cu) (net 16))
 (segment (start 23.1 20.4) (end 25 18.5) (width 0.768) (layer F.Cu) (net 16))
 (segment (start 25 18.5) (end 29.25 18.5) (width 0.768) (layer F.Cu) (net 16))
 (segment (start 29.25 18.5) (end 29.75 19) (width 0.768) (layer F.Cu) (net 16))
 (segment (start 32.29 19) (end 32.29 20.21) (width 0.768) (layer F.Cu) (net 15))
 (segment (start 27.25 21.25) (end 26.5 20.5) (width 0.768) (layer F.Cu) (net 15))
 (segment (start 31.25 21.25) (end 27.25 21.25) (width 0.768) (layer F.Cu) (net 15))
 (segment (start 32.29 20.21) (end 31.25 21.25) (width 0.768) (layer F.Cu) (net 15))
 (segment (start 35.08 18.5) (end 35.08 18.58) (width 0.25) (layer F.Cu) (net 14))
 (segment (start 34.83 19) (end 34.83 19.33) (width 0.768) (layer F.Cu) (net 14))
 (segment (start 34.83 19.33) (end 36.75 21.25) (width 0.768) (layer F.Cu) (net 14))
 (segment (start 36.75 21.25) (end 40.35 21.25) (width 0.768) (layer F.Cu) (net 14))
 (segment (start 40.35 21.25) (end 40.6 21) (width 0.768) (layer F.Cu) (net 14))
 (segment (start 32.23 48) (end 32.23 48.53) (width 0.512) (layer F.Cu) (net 11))
 (segment (start 32.23 48.53) (end 33.4 49.7) (width 0.512) (layer F.Cu) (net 11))
 (segment (start 33.4 49.7) (end 40.1 49.7) (width 0.512) (layer F.Cu) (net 11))
 (segment (start 40.1 49.7) (end 44 45.8) (width 0.512) (layer F.Cu) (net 11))
 (segment (start 44 45.8) (end 44 41.9) (width 0.512) (layer F.Cu) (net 11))
 (segment (start 44 41.9) (end 43.4 41.3) (width 0.512) (layer F.Cu) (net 11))
 (segment (start 43.4 41.3) (end 41.6 41.3) (width 0.512) (layer F.Cu) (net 11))
 (segment (start 31.92 47.92) (end 31.92 47.5) (width 0.512) (layer F.Cu) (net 11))
 (segment (start 43.25 34.8) (end 43.25 40.5) (width 0.512) (layer F.Cu) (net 11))
 (segment (start 42.45 41.3) (end 41.6 41.3) (width 0.512) (layer F.Cu) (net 11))
 (segment (start 43.25 40.5) (end 42.45 41.3) (width 0.512) (layer F.Cu) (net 11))
 (segment (start 31.92 47.67) (end 31.92 47.5) (width 0.512) (layer F.Cu) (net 11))
 (segment (start 23.1 27.5) (end 23.1 31.55) (width 0.768) (layer F.Cu) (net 9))
 (segment (start 23.1 31.55) (end 23.25 31.7) (width 0.768) (layer F.Cu) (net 9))
 (segment (start 29.69 48) (end 26.25 48) (width 0.512) (layer F.Cu) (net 10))
 (segment (start 26.25 48) (end 23.25 45) (width 0.512) (layer F.Cu) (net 10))
 (segment (start 25.65 36.7) (end 24.3 36.7) (width 0.512) (layer F.Cu) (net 10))
 (segment (start 23.25 37.75) (end 23.25 45) (width 0.512) (layer F.Cu) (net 10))
 (segment (start 24.3 36.7) (end 23.25 37.75) (width 0.512) (layer F.Cu) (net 10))
 (segment (start 25.65 36.7) (end 23.95 36.7) (width 0.512) (layer F.Cu) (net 10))
 (segment (start 23.25 36) (end 23.25 33.8) (width 0.512) (layer F.Cu) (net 10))
 (segment (start 23.95 36.7) (end 23.25 36) (width 0.512) (layer F.Cu) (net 10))
 (segment (start 44 28) (end 44 31.95) (width 0.512) (layer F.Cu) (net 12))
 (segment (start 44 31.95) (end 43.25 32.7) (width 0.512) (layer F.Cu) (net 12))
 (segment (start 35.5 37.9) (end 35.5 39.5) (width 0.768) (layer F.Cu) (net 2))
 (segment (start 34.3 40.7) (end 34.3 41) (width 0.768) (layer F.Cu) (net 2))
 (segment (start 35.5 39.5) (end 34.3 40.7) (width 0.768) (layer F.Cu) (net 2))
 (segment (start 37 43.45) (end 35.95 43.45) (width 0.512) (layer F.Cu) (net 2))
 (segment (start 35.95 43.45) (end 34.5 42) (width 0.512) (layer F.Cu) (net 2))
 (segment (start 34.5 42) (end 34.3 42) (width 0.512) (layer F.Cu) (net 2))
 (segment (start 39.4 43.2) (end 37.25 43.2) (width 0.512) (layer F.Cu) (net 2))
 (segment (start 37.25 43.2) (end 37 43.45) (width 0.512) (layer F.Cu) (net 2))
 (segment (start 34.46 47.5) (end 34.46 42.16) (width 0.512) (layer F.Cu) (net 2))
 (segment (start 34.46 42.16) (end 34.3 42) (width 0.512) (layer F.Cu) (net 2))
 (segment (start 34.3 42) (end 34.3 42.05) (width 0.768) (layer F.Cu) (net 2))
 (segment (start 30.5 34.8) (end 32.05 34.8) (width 0.768) (layer F.Cu) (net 2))
 (segment (start 32.05 34.8) (end 33 35.75) (width 0.768) (layer F.Cu) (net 2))
 (segment (start 33 35.75) (end 33 37.5) (width 0.768) (layer F.Cu) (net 2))
 (segment (start 33 37.5) (end 33 40) (width 0.768) (layer F.Cu) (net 2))
 (segment (start 34.3 42) (end 34.3 41) (width 0.768) (layer F.Cu) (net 2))
 (segment (start 33.75 40) (end 33 40) (width 0.768) (layer F.Cu) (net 2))
 (segment (start 34.3 40.55) (end 33.75 40) (width 0.768) (layer F.Cu) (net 2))
 (segment (start 34.3 41) (end 34.3 40.55) (width 0.768) (layer F.Cu) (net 2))
 (segment (start 30.1 40) (end 29.25 40.85) (width 0.768) (layer F.Cu) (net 2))
 (segment (start 33 40) (end 30.1 40) (width 0.768) (layer F.Cu) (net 2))
 (segment (start 34.46 42.16) (end 34.3 42) (width 0.768) (layer F.Cu) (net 2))
 (segment (start 27.85 34.8) (end 30.5 34.8) (width 0.512) (layer F.Cu) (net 2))
 (segment (start 44 21) (end 44 20.75) (width 0.768) (layer F.Cu) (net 13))
 (segment (start 44 20.75) (end 42.25 19) (width 0.768) (layer F.Cu) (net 13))
 (segment (start 42.25 19) (end 37.37 19) (width 0.768) (layer F.Cu) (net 13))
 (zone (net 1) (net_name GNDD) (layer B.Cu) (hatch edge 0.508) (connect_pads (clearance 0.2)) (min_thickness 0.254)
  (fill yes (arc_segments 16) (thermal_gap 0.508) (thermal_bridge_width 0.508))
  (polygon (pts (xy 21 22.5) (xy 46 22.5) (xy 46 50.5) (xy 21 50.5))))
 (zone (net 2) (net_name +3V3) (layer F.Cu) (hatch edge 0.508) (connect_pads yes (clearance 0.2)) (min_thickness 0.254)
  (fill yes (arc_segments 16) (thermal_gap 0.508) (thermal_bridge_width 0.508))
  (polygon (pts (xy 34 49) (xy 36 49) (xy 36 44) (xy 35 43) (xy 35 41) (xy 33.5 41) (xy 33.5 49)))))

